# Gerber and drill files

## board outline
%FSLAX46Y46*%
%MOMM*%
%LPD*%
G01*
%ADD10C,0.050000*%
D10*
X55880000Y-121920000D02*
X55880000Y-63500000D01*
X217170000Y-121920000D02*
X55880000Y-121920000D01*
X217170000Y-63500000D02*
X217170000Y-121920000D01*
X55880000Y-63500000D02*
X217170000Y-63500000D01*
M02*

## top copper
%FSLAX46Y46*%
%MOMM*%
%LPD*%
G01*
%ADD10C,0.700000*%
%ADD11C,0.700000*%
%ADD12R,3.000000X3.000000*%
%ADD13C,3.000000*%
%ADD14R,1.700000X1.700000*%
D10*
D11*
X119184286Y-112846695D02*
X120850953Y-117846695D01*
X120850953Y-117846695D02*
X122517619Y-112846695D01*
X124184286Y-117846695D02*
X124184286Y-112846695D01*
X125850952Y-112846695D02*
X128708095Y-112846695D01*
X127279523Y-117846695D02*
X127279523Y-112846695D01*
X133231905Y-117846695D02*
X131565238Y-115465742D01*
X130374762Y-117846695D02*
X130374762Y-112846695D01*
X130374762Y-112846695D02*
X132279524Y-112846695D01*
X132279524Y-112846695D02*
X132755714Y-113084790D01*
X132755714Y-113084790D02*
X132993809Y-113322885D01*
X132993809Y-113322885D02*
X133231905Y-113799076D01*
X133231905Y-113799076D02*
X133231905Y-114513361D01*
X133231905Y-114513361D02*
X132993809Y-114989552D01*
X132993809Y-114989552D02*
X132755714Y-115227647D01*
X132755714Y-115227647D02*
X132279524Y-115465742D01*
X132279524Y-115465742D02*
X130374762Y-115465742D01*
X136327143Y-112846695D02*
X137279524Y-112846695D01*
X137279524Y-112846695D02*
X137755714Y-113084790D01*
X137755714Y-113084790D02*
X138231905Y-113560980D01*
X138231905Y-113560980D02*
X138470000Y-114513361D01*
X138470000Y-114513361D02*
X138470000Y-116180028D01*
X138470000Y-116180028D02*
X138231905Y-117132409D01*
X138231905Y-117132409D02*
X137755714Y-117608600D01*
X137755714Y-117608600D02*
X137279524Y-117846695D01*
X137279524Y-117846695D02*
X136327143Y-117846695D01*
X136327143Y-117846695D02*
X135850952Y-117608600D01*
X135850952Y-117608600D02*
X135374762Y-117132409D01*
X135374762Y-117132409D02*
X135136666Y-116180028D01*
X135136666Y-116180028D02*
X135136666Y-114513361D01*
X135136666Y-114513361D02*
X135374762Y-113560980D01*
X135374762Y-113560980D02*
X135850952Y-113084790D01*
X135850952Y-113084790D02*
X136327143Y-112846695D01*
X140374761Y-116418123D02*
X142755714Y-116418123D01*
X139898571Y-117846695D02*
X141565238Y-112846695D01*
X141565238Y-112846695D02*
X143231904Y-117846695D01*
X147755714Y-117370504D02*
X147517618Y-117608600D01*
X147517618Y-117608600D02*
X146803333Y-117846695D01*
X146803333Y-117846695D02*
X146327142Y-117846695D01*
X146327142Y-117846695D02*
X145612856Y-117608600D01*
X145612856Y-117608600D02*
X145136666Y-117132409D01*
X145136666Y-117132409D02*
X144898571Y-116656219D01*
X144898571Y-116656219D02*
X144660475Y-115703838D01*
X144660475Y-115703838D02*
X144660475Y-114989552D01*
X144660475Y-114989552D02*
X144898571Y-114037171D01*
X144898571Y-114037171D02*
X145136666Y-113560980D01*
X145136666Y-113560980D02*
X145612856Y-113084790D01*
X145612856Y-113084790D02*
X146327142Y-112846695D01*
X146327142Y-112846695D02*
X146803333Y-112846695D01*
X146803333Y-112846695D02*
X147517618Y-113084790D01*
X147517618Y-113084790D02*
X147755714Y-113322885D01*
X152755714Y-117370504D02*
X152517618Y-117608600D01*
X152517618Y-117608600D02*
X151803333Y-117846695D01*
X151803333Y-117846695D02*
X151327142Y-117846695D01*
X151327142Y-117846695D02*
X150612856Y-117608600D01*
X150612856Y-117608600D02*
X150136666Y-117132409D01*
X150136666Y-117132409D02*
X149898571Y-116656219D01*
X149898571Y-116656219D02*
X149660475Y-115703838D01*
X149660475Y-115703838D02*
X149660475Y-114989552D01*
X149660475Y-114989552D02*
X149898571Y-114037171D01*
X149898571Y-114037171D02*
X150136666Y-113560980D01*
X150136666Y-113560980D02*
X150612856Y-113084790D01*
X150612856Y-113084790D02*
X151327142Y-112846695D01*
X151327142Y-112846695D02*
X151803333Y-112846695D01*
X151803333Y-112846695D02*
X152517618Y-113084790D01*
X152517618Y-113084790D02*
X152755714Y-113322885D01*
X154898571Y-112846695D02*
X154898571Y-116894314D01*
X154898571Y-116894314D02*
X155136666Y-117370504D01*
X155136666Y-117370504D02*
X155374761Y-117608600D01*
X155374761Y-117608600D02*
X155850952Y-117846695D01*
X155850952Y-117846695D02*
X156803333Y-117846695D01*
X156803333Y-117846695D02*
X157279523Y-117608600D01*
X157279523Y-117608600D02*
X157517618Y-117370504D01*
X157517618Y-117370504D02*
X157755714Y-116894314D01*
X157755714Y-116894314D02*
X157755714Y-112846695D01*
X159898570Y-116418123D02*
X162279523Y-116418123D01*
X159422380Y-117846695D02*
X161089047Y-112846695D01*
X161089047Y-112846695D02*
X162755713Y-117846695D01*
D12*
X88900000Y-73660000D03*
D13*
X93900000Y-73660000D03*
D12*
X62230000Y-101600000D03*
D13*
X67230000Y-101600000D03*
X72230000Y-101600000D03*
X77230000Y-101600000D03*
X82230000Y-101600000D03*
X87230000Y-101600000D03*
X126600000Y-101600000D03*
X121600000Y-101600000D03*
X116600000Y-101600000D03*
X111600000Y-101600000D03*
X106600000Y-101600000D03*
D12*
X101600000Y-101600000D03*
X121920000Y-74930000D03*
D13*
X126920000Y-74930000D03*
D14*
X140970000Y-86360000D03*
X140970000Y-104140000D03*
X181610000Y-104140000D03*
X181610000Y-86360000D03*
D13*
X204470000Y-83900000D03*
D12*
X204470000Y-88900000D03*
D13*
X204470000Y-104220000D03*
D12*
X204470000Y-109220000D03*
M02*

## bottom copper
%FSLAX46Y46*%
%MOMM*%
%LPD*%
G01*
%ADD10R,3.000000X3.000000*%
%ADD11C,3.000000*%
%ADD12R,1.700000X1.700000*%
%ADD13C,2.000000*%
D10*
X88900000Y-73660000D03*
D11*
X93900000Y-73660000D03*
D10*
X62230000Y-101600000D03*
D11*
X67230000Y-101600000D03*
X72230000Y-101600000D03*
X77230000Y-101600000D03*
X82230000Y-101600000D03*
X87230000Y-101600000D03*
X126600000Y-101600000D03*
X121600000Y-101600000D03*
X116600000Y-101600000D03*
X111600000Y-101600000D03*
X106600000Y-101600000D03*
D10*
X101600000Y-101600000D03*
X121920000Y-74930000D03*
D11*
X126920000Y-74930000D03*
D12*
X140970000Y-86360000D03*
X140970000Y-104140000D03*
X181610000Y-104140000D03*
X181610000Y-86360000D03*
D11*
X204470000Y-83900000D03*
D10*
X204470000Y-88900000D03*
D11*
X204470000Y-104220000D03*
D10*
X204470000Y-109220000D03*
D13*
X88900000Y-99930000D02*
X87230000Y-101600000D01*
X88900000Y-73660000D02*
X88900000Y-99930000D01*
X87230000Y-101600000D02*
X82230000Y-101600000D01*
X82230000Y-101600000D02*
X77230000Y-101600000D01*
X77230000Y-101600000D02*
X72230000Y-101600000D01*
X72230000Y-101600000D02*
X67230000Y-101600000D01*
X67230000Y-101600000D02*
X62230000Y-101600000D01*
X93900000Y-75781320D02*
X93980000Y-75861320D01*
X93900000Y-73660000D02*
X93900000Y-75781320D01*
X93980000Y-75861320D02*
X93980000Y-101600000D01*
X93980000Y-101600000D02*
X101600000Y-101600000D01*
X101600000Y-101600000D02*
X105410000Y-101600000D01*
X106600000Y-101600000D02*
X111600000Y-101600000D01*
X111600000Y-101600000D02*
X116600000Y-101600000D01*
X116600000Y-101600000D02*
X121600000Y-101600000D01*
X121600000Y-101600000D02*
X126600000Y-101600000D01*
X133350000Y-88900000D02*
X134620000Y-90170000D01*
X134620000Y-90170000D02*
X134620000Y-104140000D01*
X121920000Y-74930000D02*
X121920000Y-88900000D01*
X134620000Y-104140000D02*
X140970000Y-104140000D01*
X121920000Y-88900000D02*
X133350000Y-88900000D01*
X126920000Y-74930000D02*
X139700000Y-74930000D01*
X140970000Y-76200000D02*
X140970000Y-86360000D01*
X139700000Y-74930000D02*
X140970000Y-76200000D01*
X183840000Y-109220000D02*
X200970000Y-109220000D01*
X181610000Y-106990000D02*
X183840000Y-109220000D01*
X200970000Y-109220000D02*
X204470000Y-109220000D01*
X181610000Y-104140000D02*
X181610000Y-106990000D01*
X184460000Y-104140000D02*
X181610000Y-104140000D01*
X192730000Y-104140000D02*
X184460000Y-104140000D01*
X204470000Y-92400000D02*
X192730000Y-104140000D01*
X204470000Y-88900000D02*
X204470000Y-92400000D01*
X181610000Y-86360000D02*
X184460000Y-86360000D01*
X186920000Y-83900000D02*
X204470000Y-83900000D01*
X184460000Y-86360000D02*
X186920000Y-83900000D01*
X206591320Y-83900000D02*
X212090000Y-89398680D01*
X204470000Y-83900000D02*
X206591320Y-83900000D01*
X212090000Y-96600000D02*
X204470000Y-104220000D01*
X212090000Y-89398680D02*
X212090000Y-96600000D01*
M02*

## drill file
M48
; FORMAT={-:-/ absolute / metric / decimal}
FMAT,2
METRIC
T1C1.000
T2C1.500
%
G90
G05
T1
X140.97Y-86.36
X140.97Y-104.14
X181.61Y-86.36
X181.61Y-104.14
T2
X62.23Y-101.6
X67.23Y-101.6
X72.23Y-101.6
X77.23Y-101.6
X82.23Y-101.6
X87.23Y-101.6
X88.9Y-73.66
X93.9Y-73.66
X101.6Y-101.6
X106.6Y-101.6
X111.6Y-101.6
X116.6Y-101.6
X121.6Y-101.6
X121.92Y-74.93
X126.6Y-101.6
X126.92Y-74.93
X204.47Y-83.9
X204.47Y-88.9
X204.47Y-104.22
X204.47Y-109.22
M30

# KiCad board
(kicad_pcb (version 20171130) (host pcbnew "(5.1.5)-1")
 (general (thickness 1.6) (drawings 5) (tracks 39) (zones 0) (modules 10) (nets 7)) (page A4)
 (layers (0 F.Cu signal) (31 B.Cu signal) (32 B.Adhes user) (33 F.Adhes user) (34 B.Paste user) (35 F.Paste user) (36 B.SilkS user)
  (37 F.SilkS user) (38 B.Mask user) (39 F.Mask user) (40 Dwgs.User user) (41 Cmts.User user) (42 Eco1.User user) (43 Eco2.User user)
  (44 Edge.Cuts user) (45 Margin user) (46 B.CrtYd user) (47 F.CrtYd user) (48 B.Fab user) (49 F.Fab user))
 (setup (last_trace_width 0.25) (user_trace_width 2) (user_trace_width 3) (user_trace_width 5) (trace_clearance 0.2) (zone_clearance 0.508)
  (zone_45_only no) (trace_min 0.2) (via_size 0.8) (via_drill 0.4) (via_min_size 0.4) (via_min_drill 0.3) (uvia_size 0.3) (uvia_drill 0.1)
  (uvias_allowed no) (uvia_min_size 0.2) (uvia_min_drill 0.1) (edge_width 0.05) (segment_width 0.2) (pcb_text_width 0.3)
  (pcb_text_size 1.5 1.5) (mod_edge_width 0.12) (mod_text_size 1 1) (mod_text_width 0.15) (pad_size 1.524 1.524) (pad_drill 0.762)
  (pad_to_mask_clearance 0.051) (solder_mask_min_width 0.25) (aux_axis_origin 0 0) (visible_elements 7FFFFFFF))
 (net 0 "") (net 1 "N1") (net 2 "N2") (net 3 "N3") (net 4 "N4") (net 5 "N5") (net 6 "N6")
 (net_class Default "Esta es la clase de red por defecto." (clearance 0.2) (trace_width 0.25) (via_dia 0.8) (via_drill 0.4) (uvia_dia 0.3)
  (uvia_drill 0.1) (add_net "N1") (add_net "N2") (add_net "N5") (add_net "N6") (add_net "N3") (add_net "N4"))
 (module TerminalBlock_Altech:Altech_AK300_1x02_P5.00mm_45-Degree (layer F.Cu) (at 88.9 73.66)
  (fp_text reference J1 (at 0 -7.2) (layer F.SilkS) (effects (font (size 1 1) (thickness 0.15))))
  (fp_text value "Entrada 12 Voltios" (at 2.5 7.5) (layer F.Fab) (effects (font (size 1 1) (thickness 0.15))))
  (pad 1 thru_hole rect (at 0 0) (size 3 3) (drill 1.5) (layers *.Cu *.Mask) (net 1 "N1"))
  (pad 2 thru_hole circle (at 5 0) (size 3 3) (drill 1.5) (layers *.Cu *.Mask) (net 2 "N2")))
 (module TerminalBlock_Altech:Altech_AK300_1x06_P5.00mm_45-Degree (layer F.Cu) (at 62.23 101.6)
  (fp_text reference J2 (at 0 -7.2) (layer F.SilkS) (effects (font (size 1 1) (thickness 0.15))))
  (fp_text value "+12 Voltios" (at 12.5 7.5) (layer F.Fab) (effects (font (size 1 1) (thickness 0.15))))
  (pad 1 thru_hole rect (at 0 0) (size 3 3) (drill 1.5) (layers *.Cu *.Mask) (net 1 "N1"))
  (pad 2 thru_hole circle (at 5 0) (size 3 3) (drill 1.5) (layers *.Cu *.Mask) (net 1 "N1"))
  (pad 3 thru_hole circle (at 10 0) (size 3 3) (drill 1.5) (layers *.Cu *.Mask) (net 1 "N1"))
  (pad 4 thru_hole circle (at 15 0) (size 3 3) (drill 1.5) (layers *.Cu *.Mask) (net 1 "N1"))
  (pad 5 thru_hole circle (at 20 0) (size 3 3) (drill 1.5) (layers *.Cu *.Mask) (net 1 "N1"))
  (pad 6 thru_hole circle (at 25 0) (size 3 3) (drill 1.5) (layers *.Cu *.Mask) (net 1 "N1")))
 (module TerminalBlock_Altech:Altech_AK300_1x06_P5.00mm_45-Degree (layer F.Cu) (at 101.6 101.6)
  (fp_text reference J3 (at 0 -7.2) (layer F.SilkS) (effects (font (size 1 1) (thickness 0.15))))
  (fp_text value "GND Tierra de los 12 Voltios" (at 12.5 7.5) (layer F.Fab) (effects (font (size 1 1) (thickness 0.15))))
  (pad 6 thru_hole circle (at 25 0) (size 3 3) (drill 1.5) (layers *.Cu *.Mask) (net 2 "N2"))
  (pad 5 thru_hole circle (at 20 0) (size 3 3) (drill 1.5) (layers *.Cu *.Mask) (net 2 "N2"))
  (pad 4 thru_hole circle (at 15 0) (size 3 3) (drill 1.5) (layers *.Cu *.Mask) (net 2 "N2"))
  (pad 3 thru_hole circle (at 10 0) (size 3 3) (drill 1.5) (layers *.Cu *.Mask) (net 2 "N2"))
  (pad 2 thru_hole circle (at 5 0) (size 3 3) (drill 1.5) (layers *.Cu *.Mask) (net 2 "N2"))
  (pad 1 thru_hole rect (at 0 0) (size 3 3) (drill 1.5) (layers *.Cu *.Mask) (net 2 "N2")))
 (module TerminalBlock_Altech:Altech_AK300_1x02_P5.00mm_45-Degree (layer F.Cu) (at 121.92 74.93)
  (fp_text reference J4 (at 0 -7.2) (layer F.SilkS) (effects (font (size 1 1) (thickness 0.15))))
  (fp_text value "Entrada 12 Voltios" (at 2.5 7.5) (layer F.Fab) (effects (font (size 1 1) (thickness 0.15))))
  (pad 1 thru_hole rect (at 0 0) (size 3 3) (drill 1.5) (layers *.Cu *.Mask) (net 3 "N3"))
  (pad 2 thru_hole circle (at 5 0) (size 3 3) (drill 1.5) (layers *.Cu *.Mask) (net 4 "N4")))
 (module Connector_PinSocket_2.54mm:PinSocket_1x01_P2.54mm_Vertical (layer F.Cu) (at 140.97 86.36)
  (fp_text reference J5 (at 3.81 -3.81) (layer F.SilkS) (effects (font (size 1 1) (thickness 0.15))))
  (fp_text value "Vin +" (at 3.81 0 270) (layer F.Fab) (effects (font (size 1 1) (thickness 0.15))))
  (pad 1 thru_hole rect (at 0 0) (size 1.7 1.7) (drill 1) (layers *.Cu *.Mask) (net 4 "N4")))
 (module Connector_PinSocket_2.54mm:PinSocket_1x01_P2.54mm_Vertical (layer F.Cu) (at 140.97 104.14)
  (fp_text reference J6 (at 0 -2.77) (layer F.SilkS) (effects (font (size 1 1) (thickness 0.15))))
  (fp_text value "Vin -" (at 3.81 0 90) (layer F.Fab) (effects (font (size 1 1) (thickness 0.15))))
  (pad 1 thru_hole rect (at 0 0) (size 1.7 1.7) (drill 1) (layers *.Cu *.Mask) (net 3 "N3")))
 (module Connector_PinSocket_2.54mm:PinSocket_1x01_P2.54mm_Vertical (layer F.Cu) (at 181.61 104.14)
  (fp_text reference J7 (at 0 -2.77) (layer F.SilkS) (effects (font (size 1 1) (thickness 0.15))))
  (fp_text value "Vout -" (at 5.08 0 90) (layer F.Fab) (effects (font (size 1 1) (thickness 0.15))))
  (pad 1 thru_hole rect (at 0 0) (size 1.7 1.7) (drill 1) (layers *.Cu *.Mask) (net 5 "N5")))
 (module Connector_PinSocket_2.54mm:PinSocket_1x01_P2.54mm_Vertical (layer F.Cu) (at 181.61 86.36)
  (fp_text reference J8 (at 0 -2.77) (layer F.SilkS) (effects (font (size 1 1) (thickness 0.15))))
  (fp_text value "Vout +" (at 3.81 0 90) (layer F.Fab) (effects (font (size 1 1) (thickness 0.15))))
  (pad 1 thru_hole rect (at 0 0) (size 1.7 1.7) (drill 1) (layers *.Cu *.Mask) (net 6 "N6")))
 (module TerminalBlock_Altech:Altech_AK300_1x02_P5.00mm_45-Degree (layer F.Cu) (at 204.47 88.9 90)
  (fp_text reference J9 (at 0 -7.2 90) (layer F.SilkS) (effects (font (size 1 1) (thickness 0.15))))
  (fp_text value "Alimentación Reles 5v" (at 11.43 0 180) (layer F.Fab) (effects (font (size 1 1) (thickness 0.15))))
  (pad 2 thru_hole circle (at 5 0 90) (size 3 3) (drill 1.5) (layers *.Cu *.Mask) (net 6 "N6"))
  (pad 1 thru_hole rect (at 0 0 90) (size 3 3) (drill 1.5) (layers *.Cu *.Mask) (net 5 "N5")))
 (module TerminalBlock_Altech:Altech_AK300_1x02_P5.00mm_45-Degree (layer F.Cu) (at 204.47 109.22 90)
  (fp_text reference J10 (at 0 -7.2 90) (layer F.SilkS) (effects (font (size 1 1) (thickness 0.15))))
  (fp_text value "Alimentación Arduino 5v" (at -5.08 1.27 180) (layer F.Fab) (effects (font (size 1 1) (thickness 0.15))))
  (pad 2 thru_hole circle (at 5 0 90) (size 3 3) (drill 1.5) (layers *.Cu *.Mask) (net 6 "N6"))
  (pad 1 thru_hole rect (at 0 0 90) (size 3 3) (drill 1.5) (layers *.Cu *.Mask) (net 5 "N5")))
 (gr_line (start 55.88 121.92) (end 55.88 63.5) (layer Edge.Cuts) (width 0.05))
 (gr_line (start 217.17 121.92) (end 55.88 121.92) (layer Edge.Cuts) (width 0.05))
 (gr_line (start 217.17 63.5) (end 217.17 121.92) (layer Edge.Cuts) (width 0.05))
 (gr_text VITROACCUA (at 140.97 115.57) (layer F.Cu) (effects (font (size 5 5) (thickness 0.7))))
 (gr_line (start 55.88 63.5) (end 217.17 63.5) (layer Edge.Cuts) (width 0.05))
 (segment (start 88.9 99.93) (end 87.23 101.6) (width 2) (layer B.Cu) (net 1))
 (segment (start 88.9 73.66) (end 88.9 99.93) (width 2) (layer B.Cu) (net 1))
 (segment (start 87.23 101.6) (end 82.23 101.6) (width 2) (layer B.Cu) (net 1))
 (segment (start 82.23 101.6) (end 77.23 101.6) (width 2) (layer B.Cu) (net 1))
 (segment (start 77.23 101.6) (end 72.23 101.6) (width 2) (layer B.Cu) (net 1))
 (segment (start 72.23 101.6) (end 67.23 101.6) (width 2) (layer B.Cu) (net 1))
 (segment (start 67.23 101.6) (end 62.23 101.6) (width 2) (layer B.Cu) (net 1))
 (segment (start 93.9 75.78132) (end 93.98 75.86132) (width 2) (layer B.Cu) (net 2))
 (segment (start 93.9 73.66) (end 93.9 75.78132) (width 2) (layer B.Cu) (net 2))
 (segment (start 93.98 75.86132) (end 93.98 101.6) (width 2) (layer B.Cu) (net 2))
 (segment (start 93.98 101.6) (end 101.6 101.6) (width 2) (layer B.Cu) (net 2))
 (segment (start 101.6 101.6) (end 105.41 101.6) (width 2) (layer B.Cu) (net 2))
 (segment (start 106.6 101.6) (end 111.6 101.6) (width 2) (layer B.Cu) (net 2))
 (segment (start 111.6 101.6) (end 116.6 101.6) (width 2) (layer B.Cu) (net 2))
 (segment (start 116.6 101.6) (end 121.6 101.6) (width 2) (layer B.Cu) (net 2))
 (segment (start 121.6 101.6) (end 126.6 101.6) (width 2) (layer B.Cu) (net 2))
 (segment (start 133.35 88.9) (end 134.62 90.17) (width 2) (layer B.Cu) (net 3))
 (segment (start 134.62 90.17) (end 134.62 104.14) (width 2) (layer B.Cu) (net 3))
 (segment (start 121.92 74.93) (end 121.92 88.9) (width 2) (layer B.Cu) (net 3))
 (segment (start 134.62 104.14) (end 140.97 104.14) (width 2) (layer B.Cu) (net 3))
 (segment (start 121.92 88.9) (end 133.35 88.9) (width 2) (layer B.Cu) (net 3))
 (segment (start 126.92 74.93) (end 139.7 74.93) (width 2) (layer B.Cu) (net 4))
 (segment (start 140.97 76.2) (end 140.97 86.36) (width 2) (layer B.Cu) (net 4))
 (segment (start 139.7 74.93) (end 140.97 76.2) (width 2) (layer B.Cu) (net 4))
 (segment (start 183.84 109.22) (end 200.97 109.22) (width 2) (layer B.Cu) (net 5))
 (segment (start 181.61 106.99) (end 183.84 109.22) (width 2) (layer B.Cu) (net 5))
 (segment (start 200.97 109.22) (end 204.47 109.22) (width 2) (layer B.Cu) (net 5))
 (segment (start 181.61 104.14) (end 181.61 106.99) (width 2) (layer B.Cu) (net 5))
 (segment (start 184.46 104.14) (end 181.61 104.14) (width 2) (layer B.Cu) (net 5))
 (segment (start 192.73 104.14) (end 184.46 104.14) (width 2) (layer B.Cu) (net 5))
 (segment (start 204.47 92.4) (end 192.73 104.14) (width 2) (layer B.Cu) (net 5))
 (segment (start 204.47 88.9) (end 204.47 92.4) (width 2) (layer B.Cu) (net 5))
 (segment (start 181.61 86.36) (end 184.46 86.36) (width 2) (layer B.Cu) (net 6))
 (segment (start 186.92 83.9) (end 204.47 83.9) (width 2) (layer B.Cu) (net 6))
 (segment (start 184.46 86.36) (end 186.92 83.9) (width 2) (layer B.Cu) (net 6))
 (segment (start 206.59132 83.9) (end 212.09 89.39868) (width 2) (layer B.Cu) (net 6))
 (segment (start 204.47 83.9) (end 206.59132 83.9) (width 2) (layer B.Cu) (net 6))
 (segment (start 212.09 96.6) (end 204.47 104.22) (width 2) (layer B.Cu) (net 6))
 (segment (start 212.09 89.39868) (end 212.09 96.6) (width 2) (layer B.Cu) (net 6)))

